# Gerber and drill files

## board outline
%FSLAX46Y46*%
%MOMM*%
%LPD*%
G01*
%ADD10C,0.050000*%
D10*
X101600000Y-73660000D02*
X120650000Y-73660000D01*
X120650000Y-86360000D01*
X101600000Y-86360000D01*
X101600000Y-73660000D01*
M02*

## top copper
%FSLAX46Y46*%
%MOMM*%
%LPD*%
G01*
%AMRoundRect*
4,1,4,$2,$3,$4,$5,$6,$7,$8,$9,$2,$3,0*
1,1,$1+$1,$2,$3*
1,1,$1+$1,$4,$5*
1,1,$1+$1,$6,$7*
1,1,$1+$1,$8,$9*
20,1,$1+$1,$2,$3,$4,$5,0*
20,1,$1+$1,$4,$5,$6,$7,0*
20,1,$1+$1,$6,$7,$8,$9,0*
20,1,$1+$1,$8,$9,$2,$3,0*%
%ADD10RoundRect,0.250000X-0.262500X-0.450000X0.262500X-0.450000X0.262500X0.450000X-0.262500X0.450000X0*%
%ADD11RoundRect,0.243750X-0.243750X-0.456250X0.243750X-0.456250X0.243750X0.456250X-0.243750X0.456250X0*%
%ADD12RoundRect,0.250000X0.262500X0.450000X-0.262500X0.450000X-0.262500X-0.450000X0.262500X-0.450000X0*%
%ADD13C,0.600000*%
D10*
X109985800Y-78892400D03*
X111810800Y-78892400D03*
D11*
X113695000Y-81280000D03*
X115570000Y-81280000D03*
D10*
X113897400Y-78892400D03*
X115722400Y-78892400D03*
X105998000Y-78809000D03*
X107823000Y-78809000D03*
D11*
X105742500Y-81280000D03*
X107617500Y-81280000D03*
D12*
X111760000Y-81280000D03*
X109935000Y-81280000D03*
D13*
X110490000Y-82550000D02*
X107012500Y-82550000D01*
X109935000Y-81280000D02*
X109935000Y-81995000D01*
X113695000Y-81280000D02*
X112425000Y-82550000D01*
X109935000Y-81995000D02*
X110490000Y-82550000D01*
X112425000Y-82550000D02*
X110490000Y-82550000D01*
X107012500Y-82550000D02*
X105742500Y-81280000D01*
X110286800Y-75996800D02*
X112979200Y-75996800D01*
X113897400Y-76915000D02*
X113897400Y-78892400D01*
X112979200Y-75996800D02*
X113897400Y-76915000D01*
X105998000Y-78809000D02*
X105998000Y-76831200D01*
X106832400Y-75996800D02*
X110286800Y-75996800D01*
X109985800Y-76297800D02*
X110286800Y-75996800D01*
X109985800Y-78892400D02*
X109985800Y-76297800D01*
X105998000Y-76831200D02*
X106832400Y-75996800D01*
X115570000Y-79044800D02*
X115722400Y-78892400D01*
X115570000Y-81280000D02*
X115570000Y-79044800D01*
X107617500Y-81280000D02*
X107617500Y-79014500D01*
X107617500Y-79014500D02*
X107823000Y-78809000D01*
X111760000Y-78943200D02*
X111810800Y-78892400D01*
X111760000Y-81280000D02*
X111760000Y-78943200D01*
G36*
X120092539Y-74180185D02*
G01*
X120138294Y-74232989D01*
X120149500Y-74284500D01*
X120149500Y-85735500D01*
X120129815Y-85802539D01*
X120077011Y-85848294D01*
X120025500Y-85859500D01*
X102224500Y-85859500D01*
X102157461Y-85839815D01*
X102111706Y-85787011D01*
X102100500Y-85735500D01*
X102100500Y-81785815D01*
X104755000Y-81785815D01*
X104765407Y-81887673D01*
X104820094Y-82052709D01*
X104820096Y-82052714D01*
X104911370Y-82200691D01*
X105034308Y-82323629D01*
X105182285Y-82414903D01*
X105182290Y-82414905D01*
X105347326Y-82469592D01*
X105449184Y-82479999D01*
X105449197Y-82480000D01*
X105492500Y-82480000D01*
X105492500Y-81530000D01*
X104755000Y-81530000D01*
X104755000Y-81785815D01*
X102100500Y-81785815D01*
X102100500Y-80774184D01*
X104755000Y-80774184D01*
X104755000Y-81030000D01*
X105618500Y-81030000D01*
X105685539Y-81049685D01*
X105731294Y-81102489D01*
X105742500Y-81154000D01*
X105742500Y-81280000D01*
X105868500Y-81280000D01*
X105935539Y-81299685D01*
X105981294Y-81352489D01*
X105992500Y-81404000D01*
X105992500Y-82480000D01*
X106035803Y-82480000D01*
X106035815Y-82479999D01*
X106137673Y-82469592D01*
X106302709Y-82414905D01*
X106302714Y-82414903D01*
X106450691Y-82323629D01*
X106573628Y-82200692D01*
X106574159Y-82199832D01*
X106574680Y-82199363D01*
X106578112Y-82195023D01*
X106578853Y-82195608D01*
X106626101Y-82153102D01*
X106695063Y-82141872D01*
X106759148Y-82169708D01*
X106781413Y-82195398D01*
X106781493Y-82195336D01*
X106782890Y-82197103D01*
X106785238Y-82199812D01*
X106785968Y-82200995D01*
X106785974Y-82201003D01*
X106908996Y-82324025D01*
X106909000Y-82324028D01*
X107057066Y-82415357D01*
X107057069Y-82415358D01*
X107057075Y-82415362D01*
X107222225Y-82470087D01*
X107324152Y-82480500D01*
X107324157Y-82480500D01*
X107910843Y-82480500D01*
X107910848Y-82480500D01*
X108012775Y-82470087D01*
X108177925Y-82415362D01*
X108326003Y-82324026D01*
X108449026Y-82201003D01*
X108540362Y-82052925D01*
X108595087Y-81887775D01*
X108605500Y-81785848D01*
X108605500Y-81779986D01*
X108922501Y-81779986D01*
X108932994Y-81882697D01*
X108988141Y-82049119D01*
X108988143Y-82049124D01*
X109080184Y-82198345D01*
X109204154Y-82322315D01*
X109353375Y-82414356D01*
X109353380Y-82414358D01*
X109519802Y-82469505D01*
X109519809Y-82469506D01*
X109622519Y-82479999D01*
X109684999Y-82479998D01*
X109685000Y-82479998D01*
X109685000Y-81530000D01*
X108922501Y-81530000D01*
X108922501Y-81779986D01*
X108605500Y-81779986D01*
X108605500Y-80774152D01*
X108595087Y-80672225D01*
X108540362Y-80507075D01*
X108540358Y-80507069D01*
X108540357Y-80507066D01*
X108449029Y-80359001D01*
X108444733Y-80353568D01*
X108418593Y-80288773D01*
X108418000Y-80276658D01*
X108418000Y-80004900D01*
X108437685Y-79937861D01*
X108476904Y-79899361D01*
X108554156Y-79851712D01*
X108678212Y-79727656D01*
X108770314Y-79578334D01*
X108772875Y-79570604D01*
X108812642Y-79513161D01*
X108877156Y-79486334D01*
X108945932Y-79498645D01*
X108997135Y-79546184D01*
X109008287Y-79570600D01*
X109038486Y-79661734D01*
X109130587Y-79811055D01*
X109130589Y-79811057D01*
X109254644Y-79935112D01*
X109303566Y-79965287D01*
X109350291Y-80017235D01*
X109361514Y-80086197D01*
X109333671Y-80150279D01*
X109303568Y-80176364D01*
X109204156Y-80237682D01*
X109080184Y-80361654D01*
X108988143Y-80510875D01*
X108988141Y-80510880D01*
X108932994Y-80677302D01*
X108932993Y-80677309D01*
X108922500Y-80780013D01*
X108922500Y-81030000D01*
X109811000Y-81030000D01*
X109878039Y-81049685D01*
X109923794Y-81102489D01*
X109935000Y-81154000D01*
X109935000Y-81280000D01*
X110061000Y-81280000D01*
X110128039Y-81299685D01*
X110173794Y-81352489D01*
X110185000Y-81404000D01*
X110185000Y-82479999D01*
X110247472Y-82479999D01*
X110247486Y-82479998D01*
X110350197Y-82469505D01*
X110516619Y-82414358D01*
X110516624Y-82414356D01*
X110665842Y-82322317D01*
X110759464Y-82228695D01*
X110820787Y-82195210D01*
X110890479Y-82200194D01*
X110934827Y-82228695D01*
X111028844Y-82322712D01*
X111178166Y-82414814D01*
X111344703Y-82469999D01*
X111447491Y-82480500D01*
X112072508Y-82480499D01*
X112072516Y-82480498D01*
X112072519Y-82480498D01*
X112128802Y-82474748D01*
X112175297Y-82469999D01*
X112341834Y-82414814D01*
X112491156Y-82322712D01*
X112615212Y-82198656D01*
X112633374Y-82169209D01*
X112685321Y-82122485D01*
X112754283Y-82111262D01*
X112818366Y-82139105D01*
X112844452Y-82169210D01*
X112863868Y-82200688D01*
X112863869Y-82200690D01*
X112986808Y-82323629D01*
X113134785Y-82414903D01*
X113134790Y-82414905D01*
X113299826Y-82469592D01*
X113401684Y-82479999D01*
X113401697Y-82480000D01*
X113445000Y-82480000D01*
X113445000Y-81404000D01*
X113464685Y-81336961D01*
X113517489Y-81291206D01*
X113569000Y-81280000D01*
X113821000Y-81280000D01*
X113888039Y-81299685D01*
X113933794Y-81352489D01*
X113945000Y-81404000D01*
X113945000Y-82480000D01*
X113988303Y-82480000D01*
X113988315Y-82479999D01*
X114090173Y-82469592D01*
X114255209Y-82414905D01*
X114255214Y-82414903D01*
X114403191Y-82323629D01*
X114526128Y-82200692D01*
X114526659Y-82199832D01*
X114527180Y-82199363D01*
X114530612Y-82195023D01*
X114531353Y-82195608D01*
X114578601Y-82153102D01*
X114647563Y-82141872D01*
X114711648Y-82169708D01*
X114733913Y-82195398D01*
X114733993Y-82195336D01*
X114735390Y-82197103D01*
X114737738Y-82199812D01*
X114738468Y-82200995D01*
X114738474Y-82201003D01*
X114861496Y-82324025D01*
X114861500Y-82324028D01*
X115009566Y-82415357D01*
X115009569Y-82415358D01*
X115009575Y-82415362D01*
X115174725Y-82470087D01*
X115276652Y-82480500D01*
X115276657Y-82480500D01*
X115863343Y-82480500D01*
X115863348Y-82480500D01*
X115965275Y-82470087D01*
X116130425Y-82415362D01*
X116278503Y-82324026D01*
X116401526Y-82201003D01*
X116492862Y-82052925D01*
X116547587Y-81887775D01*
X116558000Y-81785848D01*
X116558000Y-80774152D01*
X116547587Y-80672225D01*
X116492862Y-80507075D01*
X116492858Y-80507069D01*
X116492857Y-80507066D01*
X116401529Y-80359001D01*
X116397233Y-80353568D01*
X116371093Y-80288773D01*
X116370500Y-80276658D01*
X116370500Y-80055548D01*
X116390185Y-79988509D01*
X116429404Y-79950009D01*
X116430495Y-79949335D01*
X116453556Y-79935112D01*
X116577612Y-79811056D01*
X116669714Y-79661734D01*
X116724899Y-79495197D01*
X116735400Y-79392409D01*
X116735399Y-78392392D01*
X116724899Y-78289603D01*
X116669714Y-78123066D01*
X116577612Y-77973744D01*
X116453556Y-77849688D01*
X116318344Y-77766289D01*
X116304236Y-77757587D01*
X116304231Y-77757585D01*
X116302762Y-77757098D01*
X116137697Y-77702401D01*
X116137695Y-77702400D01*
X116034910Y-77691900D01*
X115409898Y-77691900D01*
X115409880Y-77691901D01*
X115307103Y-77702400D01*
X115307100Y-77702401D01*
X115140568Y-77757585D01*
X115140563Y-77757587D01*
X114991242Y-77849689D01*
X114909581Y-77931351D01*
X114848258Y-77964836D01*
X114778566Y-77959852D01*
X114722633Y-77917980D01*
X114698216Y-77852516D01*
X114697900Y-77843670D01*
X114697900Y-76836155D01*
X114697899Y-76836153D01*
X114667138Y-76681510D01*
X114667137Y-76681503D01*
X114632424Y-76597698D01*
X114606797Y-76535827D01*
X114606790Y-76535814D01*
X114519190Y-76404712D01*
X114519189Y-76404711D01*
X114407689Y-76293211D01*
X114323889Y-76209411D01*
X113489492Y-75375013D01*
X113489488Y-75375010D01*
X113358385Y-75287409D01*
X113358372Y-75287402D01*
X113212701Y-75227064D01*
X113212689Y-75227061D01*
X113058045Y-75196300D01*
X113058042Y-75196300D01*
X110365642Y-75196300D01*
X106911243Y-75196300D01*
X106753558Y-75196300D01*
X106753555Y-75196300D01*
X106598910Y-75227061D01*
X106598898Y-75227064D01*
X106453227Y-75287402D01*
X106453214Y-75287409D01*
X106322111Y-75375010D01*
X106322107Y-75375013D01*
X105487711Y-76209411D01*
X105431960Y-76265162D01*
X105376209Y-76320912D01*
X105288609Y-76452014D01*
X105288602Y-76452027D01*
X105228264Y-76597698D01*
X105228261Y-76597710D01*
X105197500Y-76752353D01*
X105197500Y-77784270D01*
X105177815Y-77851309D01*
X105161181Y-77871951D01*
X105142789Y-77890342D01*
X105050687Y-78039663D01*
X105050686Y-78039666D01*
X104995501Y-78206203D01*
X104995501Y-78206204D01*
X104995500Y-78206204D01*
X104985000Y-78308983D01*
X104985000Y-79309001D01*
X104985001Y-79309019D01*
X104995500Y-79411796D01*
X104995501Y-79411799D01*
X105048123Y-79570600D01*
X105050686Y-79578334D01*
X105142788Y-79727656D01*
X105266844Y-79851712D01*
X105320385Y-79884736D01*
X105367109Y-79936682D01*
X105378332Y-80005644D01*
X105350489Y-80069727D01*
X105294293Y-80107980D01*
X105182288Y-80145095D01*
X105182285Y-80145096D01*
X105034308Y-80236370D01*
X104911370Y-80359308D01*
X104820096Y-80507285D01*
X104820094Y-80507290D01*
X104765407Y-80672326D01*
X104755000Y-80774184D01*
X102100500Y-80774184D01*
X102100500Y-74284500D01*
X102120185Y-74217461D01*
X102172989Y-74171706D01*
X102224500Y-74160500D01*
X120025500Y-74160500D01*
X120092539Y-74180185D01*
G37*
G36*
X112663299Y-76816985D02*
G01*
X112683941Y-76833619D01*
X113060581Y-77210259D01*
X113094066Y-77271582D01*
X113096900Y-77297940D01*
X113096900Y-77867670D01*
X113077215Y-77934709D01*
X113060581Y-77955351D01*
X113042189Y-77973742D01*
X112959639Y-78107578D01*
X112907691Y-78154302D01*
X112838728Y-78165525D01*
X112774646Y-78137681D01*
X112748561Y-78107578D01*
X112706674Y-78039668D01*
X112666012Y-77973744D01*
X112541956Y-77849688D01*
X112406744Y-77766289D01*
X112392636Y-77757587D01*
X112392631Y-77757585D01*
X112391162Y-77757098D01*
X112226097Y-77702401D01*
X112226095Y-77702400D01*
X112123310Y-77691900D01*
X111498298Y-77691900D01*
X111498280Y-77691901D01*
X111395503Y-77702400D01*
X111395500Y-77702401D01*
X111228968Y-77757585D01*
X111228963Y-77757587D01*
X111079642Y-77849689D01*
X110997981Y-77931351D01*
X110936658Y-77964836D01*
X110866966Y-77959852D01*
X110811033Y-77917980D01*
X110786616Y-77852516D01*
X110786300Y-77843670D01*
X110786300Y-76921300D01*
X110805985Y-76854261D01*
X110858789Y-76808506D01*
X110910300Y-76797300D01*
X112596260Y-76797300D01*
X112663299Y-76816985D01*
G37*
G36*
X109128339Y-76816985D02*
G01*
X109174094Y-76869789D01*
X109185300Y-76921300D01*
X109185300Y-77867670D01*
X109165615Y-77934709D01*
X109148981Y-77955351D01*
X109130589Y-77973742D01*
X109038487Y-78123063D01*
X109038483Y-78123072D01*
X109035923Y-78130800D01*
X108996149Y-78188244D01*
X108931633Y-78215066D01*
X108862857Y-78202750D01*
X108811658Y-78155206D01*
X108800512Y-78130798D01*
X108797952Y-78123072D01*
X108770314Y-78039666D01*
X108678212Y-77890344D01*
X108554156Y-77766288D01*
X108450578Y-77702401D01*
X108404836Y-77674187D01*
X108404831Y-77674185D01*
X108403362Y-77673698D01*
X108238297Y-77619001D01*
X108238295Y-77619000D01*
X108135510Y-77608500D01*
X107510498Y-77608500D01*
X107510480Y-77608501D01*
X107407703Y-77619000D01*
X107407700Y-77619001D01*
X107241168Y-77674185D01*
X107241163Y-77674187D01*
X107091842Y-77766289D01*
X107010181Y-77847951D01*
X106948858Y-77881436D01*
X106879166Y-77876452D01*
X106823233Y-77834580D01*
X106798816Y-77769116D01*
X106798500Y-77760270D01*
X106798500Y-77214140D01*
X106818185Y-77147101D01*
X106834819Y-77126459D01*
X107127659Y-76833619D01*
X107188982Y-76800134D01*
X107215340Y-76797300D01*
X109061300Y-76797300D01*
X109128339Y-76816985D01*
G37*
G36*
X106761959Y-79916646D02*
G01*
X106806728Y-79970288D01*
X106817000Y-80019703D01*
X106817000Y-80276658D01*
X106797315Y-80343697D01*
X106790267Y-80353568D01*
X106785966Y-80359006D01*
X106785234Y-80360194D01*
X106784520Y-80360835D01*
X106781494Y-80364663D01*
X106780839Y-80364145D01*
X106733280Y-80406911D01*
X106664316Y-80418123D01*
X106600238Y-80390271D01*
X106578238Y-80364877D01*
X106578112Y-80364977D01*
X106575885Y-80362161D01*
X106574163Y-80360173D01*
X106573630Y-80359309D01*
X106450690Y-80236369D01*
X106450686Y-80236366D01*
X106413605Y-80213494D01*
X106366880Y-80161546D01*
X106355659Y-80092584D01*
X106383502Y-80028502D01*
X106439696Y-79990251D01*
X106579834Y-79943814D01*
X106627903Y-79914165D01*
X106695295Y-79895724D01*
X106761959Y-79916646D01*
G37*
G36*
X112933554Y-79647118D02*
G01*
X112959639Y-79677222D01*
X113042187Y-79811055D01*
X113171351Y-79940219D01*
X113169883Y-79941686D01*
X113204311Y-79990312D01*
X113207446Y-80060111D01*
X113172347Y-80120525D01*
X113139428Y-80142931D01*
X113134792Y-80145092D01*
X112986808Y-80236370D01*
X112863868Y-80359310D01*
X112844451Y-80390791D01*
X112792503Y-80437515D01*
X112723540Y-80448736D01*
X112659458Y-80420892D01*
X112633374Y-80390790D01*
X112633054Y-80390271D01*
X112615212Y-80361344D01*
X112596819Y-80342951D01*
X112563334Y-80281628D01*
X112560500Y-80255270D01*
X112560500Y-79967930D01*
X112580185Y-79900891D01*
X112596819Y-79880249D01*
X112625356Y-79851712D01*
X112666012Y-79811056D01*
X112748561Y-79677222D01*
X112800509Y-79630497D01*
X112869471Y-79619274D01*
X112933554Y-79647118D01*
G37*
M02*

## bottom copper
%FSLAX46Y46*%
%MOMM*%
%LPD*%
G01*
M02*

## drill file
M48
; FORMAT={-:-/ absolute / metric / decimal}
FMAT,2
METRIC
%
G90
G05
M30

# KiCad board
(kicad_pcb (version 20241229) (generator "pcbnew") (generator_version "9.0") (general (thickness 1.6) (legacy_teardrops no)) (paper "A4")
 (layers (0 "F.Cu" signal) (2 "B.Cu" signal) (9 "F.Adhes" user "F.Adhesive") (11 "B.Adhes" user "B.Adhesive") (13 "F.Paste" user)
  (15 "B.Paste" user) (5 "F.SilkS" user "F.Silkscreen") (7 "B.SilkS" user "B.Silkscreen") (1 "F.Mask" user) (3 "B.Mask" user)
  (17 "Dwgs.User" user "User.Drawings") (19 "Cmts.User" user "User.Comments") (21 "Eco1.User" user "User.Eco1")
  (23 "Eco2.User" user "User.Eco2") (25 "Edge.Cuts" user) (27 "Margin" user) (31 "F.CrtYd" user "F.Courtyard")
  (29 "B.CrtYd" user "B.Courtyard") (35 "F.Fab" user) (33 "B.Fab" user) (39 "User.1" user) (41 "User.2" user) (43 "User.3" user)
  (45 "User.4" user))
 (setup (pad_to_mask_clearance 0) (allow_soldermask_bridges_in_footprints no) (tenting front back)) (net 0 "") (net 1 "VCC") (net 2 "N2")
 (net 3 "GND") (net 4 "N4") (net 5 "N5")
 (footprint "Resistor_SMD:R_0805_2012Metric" (layer "F.Cu") (at 110.8983 78.8924)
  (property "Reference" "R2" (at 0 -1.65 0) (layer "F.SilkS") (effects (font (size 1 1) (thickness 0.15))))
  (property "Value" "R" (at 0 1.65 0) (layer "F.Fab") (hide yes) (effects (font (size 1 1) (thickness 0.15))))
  (pad "1" smd roundrect (at -0.9125 0) (size 1.025 1.4) (layers "F.Cu" "F.Mask" "F.Paste") (roundrect_rratio 0.243902) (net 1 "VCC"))
  (pad "2" smd roundrect (at 0.9125 0) (size 1.025 1.4) (layers "F.Cu" "F.Mask" "F.Paste") (roundrect_rratio 0.243902) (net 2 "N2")))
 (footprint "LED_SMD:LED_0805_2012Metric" (layer "F.Cu") (at 114.6325 81.28)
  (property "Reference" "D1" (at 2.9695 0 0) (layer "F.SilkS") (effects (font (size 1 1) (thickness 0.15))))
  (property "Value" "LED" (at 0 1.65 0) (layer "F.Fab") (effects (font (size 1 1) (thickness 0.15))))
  (pad "1" smd roundrect (at -0.9375 0) (size 0.975 1.4) (layers "F.Cu" "F.Mask" "F.Paste") (roundrect_rratio 0.25) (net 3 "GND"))
  (pad "2" smd roundrect (at 0.9375 0) (size 0.975 1.4) (layers "F.Cu" "F.Mask" "F.Paste") (roundrect_rratio 0.25) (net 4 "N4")))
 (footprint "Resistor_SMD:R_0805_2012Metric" (layer "F.Cu") (at 114.8099 78.8924)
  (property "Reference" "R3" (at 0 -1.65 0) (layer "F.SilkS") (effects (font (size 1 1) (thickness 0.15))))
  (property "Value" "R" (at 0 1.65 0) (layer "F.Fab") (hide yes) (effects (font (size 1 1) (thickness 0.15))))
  (pad "1" smd roundrect (at -0.9125 0) (size 1.025 1.4) (layers "F.Cu" "F.Mask" "F.Paste") (roundrect_rratio 0.243902) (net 1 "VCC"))
  (pad "2" smd roundrect (at 0.9125 0) (size 1.025 1.4) (layers "F.Cu" "F.Mask" "F.Paste") (roundrect_rratio 0.243902) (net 4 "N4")))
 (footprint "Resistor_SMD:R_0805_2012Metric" (layer "F.Cu") (at 106.9105 78.809)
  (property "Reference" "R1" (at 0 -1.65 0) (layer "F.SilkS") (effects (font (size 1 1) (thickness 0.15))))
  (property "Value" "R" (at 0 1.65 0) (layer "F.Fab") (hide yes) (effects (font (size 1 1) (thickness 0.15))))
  (pad "1" smd roundrect (at -0.9125 0) (size 1.025 1.4) (layers "F.Cu" "F.Mask" "F.Paste") (roundrect_rratio 0.243902) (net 1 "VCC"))
  (pad "2" smd roundrect (at 0.9125 0) (size 1.025 1.4) (layers "F.Cu" "F.Mask" "F.Paste") (roundrect_rratio 0.243902) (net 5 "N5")))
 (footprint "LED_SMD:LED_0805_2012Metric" (layer "F.Cu") (at 106.68 81.28)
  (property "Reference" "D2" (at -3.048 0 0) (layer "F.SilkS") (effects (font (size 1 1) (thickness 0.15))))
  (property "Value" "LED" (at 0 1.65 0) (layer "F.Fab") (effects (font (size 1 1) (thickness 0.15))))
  (pad "1" smd roundrect (at -0.9375 0) (size 0.975 1.4) (layers "F.Cu" "F.Mask" "F.Paste") (roundrect_rratio 0.25) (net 3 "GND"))
  (pad "2" smd roundrect (at 0.9375 0) (size 0.975 1.4) (layers "F.Cu" "F.Mask" "F.Paste") (roundrect_rratio 0.25) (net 5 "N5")))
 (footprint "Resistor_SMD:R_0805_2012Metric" (layer "F.Cu") (at 110.8475 81.28 180)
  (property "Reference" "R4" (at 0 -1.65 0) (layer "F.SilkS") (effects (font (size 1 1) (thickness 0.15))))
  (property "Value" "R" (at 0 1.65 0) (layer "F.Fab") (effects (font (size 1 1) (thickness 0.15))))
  (pad "1" smd roundrect (at -0.9125 0 180) (size 1.025 1.4) (layers "F.Cu" "F.Mask" "F.Paste") (roundrect_rratio 0.243902) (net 2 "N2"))
  (pad "2" smd roundrect (at 0.9125 0 180) (size 1.025 1.4) (layers "F.Cu" "F.Mask" "F.Paste") (roundrect_rratio 0.243902) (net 3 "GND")))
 (gr_rect (start 101.6 73.66) (end 120.65 86.36) (stroke (width 0.05) (type default)) (fill no) (layer "Edge.Cuts"))
 (segment (start 110.49 82.55) (end 107.0125 82.55) (width 0.6) (layer "F.Cu") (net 3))
 (segment (start 109.935 81.28) (end 109.935 81.995) (width 0.6) (layer "F.Cu") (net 3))
 (segment (start 113.695 81.28) (end 112.425 82.55) (width 0.6) (layer "F.Cu") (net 3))
 (segment (start 109.935 81.995) (end 110.49 82.55) (width 0.6) (layer "F.Cu") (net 3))
 (segment (start 112.425 82.55) (end 110.49 82.55) (width 0.6) (layer "F.Cu") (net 3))
 (segment (start 107.0125 82.55) (end 105.7425 81.28) (width 0.6) (layer "F.Cu") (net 3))
 (segment (start 110.2868 75.9968) (end 112.9792 75.9968) (width 0.6) (layer "F.Cu") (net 1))
 (segment (start 113.8974 76.915) (end 113.8974 78.8924) (width 0.6) (layer "F.Cu") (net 1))
 (segment (start 112.9792 75.9968) (end 113.8974 76.915) (width 0.6) (layer "F.Cu") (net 1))
 (segment (start 105.998 78.809) (end 105.998 76.8312) (width 0.6) (layer "F.Cu") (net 1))
 (segment (start 106.8324 75.9968) (end 110.2868 75.9968) (width 0.6) (layer "F.Cu") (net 1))
 (segment (start 109.9858 76.2978) (end 110.2868 75.9968) (width 0.6) (layer "F.Cu") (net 1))
 (segment (start 109.9858 78.8924) (end 109.9858 76.2978) (width 0.6) (layer "F.Cu") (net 1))
 (segment (start 105.998 76.8312) (end 106.8324 75.9968) (width 0.6) (layer "F.Cu") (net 1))
 (segment (start 115.57 79.0448) (end 115.7224 78.8924) (width 0.6) (layer "F.Cu") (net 4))
 (segment (start 115.57 81.28) (end 115.57 79.0448) (width 0.6) (layer "F.Cu") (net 4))
 (segment (start 107.6175 81.28) (end 107.6175 79.0145) (width 0.6) (layer "F.Cu") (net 5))
 (segment (start 107.6175 79.0145) (end 107.823 78.809) (width 0.6) (layer "F.Cu") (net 5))
 (segment (start 111.76 78.9432) (end 111.8108 78.8924) (width 0.6) (layer "F.Cu") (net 2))
 (segment (start 111.76 81.28) (end 111.76 78.9432) (width 0.6) (layer "F.Cu") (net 2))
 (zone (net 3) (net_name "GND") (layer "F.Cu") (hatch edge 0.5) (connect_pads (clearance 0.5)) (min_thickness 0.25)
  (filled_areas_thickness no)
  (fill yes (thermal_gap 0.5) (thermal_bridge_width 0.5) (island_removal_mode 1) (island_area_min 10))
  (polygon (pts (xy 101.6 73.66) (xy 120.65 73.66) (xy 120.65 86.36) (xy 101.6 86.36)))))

